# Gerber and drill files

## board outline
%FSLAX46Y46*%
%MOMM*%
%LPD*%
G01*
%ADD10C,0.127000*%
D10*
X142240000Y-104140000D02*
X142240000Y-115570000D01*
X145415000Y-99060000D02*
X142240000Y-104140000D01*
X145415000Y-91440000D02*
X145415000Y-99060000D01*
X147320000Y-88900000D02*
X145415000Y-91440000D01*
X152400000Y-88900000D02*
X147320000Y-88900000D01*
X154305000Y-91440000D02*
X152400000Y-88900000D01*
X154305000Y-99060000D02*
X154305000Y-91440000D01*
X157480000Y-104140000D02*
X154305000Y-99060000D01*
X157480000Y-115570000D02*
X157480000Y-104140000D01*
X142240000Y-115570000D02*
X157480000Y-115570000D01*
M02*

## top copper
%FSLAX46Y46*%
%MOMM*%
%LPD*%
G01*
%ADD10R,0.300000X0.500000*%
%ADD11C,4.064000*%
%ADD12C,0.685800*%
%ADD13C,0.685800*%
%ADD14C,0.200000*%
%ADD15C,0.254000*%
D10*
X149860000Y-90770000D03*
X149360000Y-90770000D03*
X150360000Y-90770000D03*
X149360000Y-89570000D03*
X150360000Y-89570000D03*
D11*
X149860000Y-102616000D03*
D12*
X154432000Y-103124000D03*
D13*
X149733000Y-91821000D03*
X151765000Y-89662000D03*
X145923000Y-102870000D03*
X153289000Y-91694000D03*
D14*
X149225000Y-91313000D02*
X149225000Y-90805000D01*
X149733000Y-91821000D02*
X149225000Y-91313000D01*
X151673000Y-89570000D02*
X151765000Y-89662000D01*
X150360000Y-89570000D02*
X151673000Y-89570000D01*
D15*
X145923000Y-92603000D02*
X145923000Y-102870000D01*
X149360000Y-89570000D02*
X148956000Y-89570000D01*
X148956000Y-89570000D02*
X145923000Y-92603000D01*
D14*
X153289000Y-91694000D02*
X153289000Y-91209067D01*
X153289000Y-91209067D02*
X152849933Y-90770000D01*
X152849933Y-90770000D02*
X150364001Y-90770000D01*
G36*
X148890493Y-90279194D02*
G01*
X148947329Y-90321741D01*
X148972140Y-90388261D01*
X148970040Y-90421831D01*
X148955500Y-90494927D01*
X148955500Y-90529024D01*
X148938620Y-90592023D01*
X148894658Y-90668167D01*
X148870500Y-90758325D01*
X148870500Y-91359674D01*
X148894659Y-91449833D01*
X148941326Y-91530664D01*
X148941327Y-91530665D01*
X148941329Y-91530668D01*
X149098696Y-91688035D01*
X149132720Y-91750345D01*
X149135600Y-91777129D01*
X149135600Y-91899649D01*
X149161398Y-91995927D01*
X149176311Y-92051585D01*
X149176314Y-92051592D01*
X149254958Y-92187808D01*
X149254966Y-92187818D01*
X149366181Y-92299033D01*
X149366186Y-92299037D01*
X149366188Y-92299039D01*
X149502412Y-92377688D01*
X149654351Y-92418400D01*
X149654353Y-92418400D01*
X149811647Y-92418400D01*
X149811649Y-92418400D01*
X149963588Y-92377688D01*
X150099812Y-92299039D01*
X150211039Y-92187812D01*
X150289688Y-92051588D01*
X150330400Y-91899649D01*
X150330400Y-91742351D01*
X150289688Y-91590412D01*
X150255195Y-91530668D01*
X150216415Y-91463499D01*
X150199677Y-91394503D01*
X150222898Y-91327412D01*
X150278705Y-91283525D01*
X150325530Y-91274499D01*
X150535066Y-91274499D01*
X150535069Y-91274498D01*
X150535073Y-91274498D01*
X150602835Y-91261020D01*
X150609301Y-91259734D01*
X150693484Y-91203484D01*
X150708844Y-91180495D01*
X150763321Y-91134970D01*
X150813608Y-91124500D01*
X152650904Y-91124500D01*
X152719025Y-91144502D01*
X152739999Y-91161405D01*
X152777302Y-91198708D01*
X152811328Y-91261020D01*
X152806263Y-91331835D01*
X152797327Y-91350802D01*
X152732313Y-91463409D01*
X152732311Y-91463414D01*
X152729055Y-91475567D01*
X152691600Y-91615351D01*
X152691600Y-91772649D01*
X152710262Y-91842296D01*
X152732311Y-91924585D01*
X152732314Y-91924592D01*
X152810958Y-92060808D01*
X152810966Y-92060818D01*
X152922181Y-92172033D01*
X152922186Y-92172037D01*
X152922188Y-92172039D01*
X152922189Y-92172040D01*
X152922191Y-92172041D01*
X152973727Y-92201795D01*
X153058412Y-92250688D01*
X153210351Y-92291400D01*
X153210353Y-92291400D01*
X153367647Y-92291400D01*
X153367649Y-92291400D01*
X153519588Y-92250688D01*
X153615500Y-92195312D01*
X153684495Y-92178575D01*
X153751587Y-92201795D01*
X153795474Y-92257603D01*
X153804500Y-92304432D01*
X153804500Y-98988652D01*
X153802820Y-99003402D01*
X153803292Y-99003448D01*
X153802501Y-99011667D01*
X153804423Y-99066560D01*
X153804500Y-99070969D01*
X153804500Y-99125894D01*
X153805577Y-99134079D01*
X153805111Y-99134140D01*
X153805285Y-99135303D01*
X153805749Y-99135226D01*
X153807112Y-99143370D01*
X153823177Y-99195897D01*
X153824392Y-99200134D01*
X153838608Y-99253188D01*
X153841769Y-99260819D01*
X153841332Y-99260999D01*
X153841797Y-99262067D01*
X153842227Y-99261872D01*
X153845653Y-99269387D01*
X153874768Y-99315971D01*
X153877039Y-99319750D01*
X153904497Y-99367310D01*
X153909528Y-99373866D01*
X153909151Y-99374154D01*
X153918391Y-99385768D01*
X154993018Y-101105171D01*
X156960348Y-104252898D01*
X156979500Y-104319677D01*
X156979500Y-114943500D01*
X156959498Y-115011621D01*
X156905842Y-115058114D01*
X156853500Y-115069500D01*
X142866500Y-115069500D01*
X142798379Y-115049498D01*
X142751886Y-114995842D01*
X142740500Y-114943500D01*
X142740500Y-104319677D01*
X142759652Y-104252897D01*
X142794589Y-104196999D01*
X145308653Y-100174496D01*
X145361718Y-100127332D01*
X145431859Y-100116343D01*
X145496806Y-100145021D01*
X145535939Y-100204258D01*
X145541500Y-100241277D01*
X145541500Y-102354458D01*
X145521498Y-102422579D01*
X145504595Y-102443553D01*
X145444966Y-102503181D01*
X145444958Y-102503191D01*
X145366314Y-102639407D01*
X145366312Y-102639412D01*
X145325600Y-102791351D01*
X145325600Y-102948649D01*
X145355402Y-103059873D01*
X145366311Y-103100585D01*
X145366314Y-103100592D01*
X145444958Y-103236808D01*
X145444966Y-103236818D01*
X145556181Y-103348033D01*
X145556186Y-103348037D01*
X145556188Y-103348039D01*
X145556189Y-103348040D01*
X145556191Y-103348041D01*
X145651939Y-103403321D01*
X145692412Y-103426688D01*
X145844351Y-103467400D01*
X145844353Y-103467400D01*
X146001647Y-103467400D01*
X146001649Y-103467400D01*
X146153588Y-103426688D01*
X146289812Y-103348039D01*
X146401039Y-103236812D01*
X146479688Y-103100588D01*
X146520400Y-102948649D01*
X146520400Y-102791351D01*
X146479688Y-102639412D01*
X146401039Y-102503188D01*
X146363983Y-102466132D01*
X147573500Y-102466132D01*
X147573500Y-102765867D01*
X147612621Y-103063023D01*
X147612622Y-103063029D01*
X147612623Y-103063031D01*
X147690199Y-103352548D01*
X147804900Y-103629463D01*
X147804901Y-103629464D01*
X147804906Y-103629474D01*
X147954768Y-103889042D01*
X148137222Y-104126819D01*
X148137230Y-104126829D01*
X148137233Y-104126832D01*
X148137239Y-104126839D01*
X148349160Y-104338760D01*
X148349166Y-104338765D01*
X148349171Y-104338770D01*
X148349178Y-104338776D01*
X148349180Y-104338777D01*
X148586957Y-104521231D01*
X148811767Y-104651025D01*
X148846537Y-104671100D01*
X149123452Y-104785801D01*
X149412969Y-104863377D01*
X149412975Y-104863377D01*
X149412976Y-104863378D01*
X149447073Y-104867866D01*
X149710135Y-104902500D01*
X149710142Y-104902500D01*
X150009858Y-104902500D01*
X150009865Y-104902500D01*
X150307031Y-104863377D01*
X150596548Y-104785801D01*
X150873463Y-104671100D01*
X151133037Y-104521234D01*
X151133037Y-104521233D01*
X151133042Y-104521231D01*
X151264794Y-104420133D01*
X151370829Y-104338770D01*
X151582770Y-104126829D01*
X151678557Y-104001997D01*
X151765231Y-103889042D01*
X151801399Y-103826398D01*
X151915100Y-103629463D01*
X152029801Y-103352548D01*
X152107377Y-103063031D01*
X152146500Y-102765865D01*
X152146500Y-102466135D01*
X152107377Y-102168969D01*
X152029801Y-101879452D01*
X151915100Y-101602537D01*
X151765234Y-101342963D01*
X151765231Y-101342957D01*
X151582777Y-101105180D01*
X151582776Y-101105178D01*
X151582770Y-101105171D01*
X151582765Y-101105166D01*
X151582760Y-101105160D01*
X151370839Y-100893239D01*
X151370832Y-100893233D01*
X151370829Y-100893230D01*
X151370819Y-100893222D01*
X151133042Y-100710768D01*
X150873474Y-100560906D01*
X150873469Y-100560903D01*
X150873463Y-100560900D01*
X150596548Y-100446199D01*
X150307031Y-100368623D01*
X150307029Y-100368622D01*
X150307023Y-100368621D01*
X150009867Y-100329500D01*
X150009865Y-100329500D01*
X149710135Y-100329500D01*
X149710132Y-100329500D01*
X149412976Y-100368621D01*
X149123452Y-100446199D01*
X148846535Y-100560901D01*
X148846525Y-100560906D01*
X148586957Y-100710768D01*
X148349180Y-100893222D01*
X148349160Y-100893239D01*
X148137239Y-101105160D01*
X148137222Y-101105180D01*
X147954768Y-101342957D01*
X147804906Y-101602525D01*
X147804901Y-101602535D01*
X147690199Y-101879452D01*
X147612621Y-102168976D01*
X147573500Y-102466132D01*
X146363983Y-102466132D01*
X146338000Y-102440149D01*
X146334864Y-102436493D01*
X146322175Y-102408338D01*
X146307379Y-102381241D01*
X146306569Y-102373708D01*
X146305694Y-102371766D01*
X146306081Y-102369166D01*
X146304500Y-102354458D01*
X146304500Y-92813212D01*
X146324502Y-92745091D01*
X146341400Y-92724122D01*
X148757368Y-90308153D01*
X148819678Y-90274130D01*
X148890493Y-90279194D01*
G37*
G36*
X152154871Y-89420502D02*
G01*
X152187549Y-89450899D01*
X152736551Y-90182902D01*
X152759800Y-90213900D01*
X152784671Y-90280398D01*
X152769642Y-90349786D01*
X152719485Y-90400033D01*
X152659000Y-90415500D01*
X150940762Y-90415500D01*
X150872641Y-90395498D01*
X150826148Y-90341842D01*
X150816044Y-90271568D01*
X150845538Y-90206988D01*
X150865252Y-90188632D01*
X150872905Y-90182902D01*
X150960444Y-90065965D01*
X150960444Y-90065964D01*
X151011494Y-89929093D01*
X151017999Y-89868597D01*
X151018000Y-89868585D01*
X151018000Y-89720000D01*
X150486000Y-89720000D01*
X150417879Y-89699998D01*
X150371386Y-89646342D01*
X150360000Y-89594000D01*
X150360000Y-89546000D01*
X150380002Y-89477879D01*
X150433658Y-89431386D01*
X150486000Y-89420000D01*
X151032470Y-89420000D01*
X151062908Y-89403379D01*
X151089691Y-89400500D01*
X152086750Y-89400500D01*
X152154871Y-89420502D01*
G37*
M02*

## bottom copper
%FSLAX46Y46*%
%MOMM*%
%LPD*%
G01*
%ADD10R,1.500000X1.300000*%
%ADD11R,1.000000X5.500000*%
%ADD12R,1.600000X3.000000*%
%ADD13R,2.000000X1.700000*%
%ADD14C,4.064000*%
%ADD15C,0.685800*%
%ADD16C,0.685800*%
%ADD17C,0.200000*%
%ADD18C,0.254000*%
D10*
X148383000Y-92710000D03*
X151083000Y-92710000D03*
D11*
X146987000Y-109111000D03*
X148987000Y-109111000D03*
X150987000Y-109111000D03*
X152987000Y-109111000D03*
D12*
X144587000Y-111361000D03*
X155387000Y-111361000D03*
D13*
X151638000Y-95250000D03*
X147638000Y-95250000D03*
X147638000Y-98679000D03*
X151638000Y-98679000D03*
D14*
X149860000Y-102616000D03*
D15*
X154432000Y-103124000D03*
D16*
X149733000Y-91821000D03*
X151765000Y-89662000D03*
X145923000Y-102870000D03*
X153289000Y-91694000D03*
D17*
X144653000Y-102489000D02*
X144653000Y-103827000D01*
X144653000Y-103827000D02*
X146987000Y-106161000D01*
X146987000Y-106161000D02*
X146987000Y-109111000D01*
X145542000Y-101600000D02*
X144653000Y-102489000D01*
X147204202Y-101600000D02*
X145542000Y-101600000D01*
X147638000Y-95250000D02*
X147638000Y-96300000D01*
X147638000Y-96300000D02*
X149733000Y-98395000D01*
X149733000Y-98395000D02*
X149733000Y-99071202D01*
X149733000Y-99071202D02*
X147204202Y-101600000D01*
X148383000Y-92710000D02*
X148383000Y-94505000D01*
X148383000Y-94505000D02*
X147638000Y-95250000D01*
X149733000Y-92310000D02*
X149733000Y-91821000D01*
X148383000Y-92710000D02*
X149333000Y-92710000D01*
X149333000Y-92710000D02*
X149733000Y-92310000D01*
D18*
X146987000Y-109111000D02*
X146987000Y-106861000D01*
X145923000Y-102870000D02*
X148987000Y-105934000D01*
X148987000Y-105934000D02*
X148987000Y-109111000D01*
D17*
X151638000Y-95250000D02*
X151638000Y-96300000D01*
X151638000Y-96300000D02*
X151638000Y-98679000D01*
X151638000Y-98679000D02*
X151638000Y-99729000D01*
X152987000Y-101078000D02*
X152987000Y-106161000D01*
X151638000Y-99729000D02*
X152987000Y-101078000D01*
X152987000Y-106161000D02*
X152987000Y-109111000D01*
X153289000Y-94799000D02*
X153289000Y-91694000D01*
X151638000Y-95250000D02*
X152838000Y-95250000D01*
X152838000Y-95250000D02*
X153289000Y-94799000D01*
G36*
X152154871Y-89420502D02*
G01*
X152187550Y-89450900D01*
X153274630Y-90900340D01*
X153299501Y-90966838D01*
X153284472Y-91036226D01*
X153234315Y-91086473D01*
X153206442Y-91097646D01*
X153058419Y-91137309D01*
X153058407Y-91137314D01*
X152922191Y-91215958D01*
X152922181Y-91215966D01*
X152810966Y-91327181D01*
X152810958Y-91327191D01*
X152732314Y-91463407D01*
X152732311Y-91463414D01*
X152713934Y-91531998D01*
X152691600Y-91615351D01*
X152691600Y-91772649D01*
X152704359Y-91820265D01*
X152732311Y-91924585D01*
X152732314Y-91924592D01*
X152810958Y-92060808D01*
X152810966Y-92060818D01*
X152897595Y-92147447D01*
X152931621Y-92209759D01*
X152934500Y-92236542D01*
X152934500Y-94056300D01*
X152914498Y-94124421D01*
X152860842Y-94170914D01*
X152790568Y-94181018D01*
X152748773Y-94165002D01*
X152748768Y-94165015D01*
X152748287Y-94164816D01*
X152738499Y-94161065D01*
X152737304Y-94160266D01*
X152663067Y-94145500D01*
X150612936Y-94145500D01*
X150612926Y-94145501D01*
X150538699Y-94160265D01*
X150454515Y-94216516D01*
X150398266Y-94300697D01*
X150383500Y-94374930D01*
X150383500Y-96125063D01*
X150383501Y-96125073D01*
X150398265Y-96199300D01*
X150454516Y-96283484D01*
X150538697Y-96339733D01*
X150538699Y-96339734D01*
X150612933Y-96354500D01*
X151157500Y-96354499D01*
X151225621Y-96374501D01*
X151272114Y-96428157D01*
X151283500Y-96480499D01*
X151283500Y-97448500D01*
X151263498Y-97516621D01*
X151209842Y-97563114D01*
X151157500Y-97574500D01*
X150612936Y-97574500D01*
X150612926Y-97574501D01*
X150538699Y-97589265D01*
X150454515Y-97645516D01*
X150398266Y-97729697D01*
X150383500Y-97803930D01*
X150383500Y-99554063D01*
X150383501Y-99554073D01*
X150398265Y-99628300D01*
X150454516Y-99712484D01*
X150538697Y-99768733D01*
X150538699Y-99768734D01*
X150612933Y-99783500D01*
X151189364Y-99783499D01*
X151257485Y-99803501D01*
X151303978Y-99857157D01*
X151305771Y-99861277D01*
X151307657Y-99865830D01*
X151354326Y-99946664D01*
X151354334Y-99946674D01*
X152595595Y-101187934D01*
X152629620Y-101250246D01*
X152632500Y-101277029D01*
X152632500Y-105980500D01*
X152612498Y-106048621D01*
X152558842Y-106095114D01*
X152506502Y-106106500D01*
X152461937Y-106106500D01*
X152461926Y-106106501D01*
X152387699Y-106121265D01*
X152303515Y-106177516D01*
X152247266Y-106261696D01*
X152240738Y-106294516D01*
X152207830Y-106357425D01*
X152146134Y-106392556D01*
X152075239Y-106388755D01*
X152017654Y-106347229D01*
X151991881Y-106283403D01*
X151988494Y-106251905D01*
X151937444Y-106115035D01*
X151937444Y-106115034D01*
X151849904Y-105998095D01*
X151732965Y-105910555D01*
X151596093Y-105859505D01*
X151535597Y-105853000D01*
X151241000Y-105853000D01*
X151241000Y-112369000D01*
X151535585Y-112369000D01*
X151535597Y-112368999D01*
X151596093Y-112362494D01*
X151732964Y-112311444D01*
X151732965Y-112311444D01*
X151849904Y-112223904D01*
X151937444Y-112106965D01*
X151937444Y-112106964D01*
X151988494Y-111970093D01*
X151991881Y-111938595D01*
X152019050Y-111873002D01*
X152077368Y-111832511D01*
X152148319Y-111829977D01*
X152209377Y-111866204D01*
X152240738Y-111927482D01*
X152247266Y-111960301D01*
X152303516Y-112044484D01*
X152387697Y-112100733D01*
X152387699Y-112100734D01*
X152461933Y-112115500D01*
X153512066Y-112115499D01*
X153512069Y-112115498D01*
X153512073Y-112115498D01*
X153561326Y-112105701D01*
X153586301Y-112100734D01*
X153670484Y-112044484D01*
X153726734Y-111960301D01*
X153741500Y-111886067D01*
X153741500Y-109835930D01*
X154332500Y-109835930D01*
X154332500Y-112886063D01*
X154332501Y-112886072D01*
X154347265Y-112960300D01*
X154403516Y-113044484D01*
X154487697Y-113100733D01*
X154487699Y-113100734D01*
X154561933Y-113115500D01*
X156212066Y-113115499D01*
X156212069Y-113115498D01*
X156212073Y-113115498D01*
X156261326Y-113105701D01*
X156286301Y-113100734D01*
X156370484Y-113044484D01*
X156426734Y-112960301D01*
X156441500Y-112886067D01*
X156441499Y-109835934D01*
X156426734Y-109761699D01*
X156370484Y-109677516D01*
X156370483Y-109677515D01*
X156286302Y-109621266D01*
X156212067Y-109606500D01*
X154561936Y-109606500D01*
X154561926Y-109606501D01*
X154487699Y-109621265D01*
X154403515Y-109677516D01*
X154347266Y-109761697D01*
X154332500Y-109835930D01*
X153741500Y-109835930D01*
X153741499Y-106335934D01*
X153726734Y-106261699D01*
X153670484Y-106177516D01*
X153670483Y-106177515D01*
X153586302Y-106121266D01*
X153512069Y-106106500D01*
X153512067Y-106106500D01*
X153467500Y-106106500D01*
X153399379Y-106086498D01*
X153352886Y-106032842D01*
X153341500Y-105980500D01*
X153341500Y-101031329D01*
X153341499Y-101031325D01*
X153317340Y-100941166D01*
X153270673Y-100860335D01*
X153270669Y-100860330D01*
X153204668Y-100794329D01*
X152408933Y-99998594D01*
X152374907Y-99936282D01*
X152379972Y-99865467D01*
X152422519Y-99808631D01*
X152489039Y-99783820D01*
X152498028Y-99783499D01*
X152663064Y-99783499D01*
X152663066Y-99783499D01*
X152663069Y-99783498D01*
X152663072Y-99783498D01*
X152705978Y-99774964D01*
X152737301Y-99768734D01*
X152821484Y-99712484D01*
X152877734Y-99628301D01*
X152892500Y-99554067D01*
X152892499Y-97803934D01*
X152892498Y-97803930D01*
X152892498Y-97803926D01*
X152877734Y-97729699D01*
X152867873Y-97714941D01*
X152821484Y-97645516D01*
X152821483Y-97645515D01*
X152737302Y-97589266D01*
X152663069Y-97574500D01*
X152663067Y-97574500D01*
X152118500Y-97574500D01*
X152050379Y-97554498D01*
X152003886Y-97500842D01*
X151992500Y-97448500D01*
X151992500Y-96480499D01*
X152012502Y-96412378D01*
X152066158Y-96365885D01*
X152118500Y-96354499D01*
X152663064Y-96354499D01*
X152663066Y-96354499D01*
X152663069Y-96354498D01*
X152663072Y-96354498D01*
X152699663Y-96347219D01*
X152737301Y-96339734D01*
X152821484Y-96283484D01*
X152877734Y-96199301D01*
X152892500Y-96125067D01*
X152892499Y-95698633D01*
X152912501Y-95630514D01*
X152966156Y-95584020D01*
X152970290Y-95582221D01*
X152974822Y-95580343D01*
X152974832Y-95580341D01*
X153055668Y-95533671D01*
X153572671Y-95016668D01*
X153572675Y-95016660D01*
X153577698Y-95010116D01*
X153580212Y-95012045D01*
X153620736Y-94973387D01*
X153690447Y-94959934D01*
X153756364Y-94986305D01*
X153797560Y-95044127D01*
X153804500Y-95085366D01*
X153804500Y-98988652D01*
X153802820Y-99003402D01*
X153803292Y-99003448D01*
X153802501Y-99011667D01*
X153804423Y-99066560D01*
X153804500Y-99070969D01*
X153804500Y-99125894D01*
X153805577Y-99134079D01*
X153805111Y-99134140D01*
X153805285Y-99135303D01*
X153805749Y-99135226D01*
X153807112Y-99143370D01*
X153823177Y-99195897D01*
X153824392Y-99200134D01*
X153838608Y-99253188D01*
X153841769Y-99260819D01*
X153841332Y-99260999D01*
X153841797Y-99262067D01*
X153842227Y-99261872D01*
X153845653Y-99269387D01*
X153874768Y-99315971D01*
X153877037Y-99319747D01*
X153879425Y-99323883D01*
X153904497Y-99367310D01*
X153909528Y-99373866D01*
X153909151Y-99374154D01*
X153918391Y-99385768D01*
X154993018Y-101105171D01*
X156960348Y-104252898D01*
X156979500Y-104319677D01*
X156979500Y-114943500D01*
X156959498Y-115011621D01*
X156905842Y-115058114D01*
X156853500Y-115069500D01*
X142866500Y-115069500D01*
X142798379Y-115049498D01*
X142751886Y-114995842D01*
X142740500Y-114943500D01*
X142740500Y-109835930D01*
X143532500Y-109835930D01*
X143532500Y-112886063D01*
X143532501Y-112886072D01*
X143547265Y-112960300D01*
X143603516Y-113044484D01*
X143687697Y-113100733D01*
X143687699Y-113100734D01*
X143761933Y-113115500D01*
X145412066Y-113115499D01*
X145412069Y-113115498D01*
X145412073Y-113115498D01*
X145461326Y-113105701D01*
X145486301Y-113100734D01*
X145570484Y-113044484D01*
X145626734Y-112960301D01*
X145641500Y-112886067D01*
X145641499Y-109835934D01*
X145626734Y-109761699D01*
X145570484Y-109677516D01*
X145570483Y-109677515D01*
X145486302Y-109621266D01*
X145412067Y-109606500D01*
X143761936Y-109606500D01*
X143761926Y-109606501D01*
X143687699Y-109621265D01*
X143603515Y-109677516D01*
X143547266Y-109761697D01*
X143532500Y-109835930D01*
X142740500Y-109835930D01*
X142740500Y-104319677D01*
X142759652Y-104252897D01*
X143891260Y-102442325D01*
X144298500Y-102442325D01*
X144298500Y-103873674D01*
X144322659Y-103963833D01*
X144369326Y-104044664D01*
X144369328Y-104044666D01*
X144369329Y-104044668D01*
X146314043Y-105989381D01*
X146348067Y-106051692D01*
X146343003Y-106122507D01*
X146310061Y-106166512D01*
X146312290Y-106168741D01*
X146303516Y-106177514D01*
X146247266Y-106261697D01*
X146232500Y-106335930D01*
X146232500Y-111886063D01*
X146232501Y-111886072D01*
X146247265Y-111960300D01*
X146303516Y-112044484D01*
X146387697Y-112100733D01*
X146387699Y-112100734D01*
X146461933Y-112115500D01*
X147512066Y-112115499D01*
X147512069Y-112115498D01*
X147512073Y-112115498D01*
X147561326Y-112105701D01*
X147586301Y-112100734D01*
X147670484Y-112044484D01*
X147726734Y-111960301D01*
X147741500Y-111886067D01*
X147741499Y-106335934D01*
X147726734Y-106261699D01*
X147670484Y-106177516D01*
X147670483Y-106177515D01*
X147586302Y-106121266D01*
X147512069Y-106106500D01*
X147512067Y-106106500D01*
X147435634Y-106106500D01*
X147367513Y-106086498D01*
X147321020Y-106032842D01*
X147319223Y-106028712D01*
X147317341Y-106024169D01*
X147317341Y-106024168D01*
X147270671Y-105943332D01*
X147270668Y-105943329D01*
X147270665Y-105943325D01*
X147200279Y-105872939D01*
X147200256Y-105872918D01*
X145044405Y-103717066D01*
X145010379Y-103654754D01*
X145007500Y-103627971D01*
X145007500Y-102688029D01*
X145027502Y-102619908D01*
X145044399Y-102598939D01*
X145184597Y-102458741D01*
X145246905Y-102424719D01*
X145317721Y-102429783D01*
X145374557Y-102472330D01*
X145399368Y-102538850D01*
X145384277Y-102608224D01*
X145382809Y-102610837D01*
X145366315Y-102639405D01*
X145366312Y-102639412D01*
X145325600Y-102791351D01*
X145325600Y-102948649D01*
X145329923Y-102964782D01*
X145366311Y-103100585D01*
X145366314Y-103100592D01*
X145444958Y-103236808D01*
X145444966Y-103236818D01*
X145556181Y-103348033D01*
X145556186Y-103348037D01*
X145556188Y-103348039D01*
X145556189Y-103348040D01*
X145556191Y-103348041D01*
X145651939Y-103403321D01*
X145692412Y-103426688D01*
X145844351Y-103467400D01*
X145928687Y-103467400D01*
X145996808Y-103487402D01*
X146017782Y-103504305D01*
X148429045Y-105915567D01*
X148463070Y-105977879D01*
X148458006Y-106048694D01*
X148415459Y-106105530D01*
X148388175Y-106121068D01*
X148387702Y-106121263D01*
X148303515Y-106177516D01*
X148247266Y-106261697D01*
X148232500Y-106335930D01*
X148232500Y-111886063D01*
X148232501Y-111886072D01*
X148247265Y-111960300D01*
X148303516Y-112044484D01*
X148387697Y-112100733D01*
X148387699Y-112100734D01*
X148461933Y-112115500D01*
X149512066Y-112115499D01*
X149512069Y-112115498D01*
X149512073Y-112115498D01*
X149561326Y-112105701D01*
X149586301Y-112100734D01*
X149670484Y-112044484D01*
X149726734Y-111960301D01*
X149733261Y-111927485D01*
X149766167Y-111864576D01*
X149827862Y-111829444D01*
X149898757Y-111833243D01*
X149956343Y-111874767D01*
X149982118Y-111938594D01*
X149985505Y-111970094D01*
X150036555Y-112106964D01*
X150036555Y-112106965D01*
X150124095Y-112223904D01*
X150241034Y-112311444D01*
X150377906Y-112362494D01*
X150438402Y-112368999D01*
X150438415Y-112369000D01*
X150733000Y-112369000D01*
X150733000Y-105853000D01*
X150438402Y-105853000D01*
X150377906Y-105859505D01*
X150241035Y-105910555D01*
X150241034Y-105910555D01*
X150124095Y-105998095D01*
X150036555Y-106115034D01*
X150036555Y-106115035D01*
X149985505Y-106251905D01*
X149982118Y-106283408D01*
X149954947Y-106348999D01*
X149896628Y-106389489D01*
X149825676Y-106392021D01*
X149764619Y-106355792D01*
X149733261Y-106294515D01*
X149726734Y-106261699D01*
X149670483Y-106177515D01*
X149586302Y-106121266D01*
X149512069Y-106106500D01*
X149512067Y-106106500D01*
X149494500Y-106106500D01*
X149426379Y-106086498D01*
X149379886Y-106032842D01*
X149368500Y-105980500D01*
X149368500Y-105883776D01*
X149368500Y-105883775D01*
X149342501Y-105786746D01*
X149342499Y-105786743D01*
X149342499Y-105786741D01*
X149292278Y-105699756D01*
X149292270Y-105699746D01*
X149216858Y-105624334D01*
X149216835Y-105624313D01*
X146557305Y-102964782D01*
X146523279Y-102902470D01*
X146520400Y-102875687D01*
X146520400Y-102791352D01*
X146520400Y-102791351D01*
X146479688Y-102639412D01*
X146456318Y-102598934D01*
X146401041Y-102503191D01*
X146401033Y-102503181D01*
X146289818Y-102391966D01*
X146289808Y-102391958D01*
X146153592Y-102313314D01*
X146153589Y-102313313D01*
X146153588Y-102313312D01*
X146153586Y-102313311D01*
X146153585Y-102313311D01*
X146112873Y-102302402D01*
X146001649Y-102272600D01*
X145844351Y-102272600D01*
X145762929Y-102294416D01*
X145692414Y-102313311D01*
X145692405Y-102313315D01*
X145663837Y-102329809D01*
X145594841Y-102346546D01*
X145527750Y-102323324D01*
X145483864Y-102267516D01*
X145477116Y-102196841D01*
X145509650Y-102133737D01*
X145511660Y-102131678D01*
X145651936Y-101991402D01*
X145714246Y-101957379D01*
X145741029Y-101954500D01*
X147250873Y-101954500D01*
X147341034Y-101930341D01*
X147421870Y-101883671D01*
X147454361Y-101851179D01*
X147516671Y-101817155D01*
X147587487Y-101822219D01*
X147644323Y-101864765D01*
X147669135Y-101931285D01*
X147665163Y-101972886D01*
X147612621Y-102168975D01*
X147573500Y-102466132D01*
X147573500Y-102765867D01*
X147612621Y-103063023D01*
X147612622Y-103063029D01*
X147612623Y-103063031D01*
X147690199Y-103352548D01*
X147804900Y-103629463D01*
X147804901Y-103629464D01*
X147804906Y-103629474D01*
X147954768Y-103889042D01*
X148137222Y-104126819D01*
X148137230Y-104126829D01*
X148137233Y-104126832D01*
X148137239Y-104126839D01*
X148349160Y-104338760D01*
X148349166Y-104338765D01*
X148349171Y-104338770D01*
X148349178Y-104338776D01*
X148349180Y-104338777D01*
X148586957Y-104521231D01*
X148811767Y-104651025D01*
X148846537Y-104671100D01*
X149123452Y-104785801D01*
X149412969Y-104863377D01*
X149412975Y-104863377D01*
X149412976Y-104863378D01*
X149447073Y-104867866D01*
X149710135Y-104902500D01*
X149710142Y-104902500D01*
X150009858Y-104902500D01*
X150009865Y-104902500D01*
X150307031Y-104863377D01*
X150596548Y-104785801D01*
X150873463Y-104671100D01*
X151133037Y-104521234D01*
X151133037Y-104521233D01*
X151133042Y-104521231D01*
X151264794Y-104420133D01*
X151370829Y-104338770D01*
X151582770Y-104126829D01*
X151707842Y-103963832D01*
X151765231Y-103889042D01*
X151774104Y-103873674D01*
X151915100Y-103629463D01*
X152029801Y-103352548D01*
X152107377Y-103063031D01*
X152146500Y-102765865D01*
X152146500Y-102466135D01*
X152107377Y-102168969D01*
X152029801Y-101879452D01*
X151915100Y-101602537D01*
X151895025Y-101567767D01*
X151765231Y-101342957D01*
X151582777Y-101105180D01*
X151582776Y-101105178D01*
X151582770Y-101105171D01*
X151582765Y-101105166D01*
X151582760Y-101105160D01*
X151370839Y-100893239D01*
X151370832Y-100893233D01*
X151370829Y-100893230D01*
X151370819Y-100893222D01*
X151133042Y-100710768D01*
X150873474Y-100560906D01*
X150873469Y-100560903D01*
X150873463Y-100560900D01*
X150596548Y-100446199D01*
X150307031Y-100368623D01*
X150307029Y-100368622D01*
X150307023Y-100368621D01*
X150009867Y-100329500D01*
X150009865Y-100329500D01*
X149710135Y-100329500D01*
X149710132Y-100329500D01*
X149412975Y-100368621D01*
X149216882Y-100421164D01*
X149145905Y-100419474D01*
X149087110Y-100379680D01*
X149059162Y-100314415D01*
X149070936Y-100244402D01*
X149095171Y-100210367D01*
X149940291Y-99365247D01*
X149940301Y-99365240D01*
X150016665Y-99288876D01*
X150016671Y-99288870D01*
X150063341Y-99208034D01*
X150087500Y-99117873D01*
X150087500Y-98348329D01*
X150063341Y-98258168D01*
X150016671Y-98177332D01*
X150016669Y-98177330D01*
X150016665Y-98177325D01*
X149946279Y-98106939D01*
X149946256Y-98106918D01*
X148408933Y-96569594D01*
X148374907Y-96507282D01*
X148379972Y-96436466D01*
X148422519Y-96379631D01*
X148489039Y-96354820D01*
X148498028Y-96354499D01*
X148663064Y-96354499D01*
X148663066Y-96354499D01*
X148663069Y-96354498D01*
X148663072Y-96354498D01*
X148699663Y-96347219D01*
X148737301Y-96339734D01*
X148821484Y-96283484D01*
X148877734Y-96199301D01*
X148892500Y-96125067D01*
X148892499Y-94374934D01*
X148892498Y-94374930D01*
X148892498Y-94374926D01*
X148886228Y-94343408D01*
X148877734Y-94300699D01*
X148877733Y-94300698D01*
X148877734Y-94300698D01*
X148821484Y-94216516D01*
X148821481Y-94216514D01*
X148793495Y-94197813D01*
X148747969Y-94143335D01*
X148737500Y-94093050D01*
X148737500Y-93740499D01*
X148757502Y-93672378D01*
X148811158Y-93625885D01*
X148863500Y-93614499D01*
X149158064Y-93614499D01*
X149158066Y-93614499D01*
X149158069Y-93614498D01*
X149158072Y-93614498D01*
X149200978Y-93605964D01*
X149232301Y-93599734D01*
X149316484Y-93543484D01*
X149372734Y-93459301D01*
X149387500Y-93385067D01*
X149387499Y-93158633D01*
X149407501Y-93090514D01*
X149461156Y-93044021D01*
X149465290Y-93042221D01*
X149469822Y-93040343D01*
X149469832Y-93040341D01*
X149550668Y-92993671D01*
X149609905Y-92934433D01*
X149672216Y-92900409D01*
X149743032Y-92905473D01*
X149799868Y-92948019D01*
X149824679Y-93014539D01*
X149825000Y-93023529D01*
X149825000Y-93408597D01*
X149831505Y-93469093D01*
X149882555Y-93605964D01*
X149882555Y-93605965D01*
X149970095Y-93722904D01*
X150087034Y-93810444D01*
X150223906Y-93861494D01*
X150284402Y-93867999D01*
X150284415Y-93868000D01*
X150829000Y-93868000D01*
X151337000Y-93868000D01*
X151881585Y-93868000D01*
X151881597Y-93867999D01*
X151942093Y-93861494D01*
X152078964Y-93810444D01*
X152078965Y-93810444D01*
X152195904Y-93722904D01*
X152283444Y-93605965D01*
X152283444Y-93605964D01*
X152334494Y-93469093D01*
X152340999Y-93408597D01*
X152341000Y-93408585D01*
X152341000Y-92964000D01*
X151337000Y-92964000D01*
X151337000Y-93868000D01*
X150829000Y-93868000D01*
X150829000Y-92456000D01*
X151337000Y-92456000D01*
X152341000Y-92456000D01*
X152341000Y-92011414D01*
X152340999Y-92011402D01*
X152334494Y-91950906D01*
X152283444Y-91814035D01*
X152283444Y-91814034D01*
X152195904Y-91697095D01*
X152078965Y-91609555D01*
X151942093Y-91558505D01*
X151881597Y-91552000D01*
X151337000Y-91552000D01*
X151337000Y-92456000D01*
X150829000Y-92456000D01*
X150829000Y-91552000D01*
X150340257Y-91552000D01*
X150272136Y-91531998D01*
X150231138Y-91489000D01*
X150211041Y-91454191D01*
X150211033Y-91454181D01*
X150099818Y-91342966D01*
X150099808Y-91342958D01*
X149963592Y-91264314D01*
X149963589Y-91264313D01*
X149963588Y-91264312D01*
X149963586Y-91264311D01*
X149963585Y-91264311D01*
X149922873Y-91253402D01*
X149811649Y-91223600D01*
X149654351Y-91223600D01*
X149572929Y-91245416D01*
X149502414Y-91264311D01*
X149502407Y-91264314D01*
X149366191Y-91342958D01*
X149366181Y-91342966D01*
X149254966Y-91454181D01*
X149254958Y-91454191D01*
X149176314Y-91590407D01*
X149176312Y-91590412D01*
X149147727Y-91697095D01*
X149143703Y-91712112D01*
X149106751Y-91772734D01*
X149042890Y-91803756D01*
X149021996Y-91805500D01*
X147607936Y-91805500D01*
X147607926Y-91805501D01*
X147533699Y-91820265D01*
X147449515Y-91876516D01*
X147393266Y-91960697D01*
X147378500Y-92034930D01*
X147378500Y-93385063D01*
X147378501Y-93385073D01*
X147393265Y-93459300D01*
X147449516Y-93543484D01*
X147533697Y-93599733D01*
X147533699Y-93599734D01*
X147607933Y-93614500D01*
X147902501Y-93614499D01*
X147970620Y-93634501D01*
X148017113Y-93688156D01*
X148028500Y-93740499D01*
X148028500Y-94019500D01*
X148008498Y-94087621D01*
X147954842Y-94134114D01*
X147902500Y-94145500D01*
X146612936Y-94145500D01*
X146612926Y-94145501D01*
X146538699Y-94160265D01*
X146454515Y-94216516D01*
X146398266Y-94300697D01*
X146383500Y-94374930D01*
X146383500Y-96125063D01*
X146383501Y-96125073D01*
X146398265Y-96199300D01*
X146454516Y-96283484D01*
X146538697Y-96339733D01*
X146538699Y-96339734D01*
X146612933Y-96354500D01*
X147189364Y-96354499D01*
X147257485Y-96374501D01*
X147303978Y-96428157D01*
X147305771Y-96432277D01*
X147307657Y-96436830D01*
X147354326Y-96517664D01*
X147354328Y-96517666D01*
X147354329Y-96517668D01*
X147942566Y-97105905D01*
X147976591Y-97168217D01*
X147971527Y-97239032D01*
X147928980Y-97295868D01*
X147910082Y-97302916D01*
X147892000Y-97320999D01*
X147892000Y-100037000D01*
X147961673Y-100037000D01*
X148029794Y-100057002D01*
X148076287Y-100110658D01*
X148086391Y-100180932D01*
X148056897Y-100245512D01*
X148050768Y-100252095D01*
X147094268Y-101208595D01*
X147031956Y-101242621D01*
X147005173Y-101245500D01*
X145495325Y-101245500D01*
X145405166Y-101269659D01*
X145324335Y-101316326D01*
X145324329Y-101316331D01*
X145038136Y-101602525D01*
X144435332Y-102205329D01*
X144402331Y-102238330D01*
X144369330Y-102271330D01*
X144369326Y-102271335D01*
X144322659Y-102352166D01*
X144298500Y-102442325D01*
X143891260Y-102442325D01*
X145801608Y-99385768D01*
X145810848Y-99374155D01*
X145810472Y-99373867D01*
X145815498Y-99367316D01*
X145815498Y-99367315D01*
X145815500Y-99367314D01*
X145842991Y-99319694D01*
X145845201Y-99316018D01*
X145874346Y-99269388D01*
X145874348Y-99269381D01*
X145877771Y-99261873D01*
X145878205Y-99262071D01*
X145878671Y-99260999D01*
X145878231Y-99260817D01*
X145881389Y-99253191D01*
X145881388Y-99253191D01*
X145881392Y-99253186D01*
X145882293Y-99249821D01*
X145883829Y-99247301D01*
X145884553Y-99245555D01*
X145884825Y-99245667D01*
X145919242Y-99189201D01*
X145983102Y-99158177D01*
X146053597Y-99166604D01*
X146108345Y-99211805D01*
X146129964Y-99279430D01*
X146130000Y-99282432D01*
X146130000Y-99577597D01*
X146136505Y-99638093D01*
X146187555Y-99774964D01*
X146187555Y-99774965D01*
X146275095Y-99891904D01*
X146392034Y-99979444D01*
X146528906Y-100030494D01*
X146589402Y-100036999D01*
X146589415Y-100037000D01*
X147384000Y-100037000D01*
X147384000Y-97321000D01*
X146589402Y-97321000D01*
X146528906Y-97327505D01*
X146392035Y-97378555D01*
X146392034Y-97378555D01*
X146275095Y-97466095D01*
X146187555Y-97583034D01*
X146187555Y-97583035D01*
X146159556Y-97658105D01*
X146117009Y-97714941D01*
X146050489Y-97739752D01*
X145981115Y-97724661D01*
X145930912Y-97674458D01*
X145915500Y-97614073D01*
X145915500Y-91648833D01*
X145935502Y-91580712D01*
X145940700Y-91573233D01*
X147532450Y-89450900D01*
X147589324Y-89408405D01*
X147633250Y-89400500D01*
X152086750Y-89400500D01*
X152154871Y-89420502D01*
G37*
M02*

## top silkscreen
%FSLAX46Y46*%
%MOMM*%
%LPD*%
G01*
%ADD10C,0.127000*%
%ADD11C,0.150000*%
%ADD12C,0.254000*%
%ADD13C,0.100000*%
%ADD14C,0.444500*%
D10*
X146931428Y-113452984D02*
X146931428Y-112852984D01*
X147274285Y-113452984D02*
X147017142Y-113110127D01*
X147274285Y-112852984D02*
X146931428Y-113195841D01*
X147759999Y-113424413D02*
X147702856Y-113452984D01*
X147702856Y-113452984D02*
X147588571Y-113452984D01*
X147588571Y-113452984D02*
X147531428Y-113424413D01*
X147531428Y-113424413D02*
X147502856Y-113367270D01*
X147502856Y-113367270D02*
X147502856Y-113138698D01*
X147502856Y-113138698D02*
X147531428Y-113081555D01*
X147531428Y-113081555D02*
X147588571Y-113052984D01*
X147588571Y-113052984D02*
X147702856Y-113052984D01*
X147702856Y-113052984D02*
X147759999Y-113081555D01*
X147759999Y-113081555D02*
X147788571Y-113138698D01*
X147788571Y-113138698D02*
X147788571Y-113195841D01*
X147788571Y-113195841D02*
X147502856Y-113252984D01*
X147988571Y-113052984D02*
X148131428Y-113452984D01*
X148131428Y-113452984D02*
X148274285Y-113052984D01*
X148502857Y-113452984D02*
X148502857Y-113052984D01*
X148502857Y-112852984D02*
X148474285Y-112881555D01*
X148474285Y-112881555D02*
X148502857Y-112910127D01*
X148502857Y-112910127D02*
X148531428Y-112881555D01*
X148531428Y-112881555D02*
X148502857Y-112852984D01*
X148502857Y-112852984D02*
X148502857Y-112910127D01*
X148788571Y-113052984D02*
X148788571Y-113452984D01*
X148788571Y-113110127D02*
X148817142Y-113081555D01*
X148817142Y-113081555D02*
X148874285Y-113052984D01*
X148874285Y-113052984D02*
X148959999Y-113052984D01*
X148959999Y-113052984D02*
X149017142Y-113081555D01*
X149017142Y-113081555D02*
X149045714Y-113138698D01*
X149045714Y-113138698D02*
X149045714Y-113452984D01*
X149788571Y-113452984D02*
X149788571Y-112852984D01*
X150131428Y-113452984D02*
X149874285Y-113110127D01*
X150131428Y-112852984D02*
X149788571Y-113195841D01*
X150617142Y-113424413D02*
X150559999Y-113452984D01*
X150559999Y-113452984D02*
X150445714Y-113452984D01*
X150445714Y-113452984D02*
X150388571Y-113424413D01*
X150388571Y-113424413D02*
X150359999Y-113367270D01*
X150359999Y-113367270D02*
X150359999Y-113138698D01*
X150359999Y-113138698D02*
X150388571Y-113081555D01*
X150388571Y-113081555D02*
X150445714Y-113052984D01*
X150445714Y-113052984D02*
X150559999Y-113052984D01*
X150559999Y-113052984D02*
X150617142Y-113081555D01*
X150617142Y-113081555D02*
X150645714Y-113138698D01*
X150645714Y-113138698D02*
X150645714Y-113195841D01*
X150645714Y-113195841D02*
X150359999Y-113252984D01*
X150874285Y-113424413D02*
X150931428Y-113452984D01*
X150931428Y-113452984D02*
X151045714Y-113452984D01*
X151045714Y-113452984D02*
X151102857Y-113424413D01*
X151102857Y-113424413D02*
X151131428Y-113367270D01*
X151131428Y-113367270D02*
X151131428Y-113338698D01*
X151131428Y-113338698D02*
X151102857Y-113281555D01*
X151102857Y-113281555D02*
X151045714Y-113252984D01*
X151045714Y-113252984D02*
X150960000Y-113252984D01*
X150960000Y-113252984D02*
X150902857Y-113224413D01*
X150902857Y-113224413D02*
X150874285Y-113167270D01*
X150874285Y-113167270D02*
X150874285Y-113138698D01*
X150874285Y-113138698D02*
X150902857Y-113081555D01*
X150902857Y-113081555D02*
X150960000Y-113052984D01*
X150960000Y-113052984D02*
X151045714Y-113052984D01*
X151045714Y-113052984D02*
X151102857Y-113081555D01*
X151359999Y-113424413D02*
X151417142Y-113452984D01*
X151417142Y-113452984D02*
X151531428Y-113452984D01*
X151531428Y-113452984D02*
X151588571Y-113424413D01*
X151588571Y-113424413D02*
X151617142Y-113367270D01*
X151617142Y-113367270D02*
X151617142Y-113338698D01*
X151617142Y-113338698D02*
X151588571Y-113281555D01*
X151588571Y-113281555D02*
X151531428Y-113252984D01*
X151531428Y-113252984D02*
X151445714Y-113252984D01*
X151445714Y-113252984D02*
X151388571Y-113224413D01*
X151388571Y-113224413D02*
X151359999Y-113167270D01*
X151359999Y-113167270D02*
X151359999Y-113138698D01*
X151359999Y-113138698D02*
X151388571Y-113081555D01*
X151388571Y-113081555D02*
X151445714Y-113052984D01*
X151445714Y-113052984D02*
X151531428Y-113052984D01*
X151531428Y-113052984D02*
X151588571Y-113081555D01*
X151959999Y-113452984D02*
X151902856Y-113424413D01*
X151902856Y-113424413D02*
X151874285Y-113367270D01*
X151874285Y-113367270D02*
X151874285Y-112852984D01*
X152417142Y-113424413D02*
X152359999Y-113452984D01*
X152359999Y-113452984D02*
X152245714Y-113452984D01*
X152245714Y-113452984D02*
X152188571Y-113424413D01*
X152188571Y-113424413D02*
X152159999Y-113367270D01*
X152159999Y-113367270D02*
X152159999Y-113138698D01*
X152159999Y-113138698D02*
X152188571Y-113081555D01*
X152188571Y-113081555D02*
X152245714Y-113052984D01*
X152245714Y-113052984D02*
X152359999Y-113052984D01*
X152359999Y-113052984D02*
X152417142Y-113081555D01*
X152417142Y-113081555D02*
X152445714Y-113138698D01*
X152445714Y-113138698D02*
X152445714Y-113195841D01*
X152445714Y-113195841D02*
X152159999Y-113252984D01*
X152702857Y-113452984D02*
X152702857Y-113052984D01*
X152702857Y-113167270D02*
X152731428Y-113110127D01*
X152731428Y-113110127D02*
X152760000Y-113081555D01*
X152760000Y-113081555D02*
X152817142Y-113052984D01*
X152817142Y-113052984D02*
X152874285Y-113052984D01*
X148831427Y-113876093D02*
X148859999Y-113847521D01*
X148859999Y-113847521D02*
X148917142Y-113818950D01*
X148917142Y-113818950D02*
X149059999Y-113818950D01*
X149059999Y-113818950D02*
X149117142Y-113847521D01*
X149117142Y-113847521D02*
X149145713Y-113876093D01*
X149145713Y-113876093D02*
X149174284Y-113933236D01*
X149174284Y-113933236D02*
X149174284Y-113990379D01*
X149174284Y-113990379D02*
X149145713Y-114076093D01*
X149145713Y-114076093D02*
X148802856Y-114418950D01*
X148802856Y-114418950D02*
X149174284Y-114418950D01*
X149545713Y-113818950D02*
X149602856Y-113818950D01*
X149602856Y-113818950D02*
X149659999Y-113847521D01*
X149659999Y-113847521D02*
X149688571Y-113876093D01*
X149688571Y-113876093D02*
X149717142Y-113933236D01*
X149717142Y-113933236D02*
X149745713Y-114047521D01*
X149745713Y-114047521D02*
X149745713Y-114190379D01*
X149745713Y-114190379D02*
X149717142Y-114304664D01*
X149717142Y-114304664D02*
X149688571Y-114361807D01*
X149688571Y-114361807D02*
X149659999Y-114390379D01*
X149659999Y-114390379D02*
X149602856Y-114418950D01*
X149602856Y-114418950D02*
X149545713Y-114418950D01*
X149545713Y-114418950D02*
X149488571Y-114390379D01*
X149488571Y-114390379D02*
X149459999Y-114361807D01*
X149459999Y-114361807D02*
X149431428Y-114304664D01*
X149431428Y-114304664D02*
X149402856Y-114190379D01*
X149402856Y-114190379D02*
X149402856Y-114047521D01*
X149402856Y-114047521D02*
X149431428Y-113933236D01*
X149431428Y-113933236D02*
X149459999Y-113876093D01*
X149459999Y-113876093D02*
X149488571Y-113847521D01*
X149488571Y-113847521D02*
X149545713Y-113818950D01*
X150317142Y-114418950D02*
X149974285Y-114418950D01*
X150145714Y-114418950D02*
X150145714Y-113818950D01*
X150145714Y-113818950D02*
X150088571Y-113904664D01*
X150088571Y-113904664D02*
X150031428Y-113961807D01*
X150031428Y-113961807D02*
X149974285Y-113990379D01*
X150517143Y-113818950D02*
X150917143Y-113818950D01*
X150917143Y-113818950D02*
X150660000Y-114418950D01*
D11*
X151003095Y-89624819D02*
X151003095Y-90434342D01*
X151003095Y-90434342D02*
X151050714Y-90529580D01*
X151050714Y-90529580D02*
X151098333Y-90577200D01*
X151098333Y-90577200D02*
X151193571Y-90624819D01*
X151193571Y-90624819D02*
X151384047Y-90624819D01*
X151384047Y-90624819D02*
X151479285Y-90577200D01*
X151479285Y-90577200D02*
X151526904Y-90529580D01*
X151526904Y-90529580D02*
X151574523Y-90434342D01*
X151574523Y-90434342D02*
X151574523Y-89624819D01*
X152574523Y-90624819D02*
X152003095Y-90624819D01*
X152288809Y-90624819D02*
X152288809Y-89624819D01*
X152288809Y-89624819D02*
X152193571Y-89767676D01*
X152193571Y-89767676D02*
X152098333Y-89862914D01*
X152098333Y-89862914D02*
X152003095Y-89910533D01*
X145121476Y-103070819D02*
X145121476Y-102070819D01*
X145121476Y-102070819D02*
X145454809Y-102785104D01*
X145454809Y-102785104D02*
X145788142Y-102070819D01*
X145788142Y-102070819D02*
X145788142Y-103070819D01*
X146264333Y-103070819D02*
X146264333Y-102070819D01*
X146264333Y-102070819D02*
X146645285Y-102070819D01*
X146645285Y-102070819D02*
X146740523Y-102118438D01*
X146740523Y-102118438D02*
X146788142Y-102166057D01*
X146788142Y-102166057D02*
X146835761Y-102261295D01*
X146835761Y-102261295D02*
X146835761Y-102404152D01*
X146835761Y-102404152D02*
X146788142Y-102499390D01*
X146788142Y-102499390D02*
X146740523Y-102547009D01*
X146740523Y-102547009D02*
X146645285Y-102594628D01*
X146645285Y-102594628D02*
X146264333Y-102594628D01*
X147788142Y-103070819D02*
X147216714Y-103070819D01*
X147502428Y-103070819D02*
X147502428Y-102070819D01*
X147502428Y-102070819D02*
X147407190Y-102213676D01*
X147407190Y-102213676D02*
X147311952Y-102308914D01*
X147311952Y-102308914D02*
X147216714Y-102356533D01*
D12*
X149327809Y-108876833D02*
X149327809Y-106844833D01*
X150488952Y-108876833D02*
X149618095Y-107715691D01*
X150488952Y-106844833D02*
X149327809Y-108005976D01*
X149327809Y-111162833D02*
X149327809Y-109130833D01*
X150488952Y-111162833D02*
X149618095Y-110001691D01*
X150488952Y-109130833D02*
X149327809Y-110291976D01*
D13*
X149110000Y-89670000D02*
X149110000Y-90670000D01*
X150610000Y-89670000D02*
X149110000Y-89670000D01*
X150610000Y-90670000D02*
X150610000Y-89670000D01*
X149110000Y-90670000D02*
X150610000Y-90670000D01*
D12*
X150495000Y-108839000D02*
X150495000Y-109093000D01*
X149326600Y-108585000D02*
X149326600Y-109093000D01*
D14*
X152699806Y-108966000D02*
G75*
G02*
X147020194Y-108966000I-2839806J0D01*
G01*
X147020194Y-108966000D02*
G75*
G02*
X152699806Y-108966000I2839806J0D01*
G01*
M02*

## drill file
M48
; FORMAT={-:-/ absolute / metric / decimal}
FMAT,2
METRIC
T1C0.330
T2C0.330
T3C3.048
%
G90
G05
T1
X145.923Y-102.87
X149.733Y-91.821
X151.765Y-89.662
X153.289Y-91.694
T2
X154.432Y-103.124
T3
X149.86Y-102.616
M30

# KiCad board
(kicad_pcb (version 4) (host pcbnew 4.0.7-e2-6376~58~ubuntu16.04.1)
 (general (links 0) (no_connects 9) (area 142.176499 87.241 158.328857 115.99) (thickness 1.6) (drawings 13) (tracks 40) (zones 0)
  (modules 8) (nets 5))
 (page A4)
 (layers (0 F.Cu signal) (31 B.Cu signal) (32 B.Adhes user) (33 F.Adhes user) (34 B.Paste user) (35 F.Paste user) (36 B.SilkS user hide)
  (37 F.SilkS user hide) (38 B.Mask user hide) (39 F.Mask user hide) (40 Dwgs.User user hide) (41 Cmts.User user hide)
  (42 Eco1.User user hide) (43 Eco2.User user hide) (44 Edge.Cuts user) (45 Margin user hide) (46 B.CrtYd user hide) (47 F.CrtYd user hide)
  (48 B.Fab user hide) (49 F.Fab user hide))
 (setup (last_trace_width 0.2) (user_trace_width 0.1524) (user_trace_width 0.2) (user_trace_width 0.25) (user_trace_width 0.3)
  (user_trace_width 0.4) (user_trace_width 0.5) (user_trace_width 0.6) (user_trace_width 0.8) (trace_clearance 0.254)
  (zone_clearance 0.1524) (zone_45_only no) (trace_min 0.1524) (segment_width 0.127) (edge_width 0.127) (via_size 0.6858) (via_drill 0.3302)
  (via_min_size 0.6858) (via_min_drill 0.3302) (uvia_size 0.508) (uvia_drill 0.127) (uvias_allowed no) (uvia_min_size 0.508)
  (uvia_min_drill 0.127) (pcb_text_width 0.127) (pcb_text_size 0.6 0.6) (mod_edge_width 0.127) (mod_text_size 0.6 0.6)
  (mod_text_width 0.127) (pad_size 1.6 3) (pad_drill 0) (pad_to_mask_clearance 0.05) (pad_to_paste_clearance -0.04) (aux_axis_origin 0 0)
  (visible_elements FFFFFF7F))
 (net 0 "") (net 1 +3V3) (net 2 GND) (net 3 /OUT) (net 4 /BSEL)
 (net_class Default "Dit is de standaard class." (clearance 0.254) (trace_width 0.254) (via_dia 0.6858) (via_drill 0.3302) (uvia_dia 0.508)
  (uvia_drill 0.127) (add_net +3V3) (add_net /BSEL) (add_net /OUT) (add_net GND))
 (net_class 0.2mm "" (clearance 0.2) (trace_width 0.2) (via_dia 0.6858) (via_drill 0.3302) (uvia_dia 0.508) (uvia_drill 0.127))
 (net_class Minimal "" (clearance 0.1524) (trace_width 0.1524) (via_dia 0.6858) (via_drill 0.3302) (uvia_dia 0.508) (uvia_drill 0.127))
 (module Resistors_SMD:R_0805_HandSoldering (layer B.Cu) (at 149.733 92.71)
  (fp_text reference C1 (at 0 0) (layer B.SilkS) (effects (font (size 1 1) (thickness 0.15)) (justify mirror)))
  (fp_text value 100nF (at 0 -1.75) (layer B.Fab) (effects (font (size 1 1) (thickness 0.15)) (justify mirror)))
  (pad 1 smd rect (at -1.35 0) (size 1.5 1.3) (layers B.Cu B.Paste B.Mask) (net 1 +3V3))
  (pad 2 smd rect (at 1.35 0) (size 1.5 1.3) (layers B.Cu B.Paste B.Mask) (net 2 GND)))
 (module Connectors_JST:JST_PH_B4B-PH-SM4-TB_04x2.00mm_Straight (layer B.Cu) (at 149.987 110.236)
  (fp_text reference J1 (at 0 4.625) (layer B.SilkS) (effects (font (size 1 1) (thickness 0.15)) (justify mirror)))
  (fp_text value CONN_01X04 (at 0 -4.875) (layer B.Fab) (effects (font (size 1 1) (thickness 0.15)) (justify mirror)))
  (pad 1 smd rect (at -3 -1.125) (size 1 5.5) (layers B.Cu B.Paste B.Mask) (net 1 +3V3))
  (pad 2 smd rect (at -1 -1.125) (size 1 5.5) (layers B.Cu B.Paste B.Mask) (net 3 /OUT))
  (pad 3 smd rect (at 1 -1.125) (size 1 5.5) (layers B.Cu B.Paste B.Mask) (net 2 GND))
  (pad 4 smd rect (at 3 -1.125) (size 1 5.5) (layers B.Cu B.Paste B.Mask) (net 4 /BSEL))
  (pad "" smd rect (at -5.4 1.125) (size 1.6 3) (layers B.Cu B.Paste B.Mask))
  (pad "" smd rect (at 5.4 1.125) (size 1.6 3) (layers B.Cu B.Paste B.Mask)))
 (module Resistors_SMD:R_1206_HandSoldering (layer B.Cu) (at 149.638 95.25 180)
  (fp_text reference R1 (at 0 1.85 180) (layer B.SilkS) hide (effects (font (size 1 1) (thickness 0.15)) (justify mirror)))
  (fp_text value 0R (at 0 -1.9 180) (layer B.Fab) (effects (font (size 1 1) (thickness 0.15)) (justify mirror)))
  (pad 1 smd rect (at -2 0 180) (size 2 1.7) (layers B.Cu B.Paste B.Mask) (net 4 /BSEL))
  (pad 2 smd rect (at 2 0 180) (size 2 1.7) (layers B.Cu B.Paste B.Mask) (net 1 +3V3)))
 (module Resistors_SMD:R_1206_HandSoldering (layer B.Cu) (at 149.638 98.679)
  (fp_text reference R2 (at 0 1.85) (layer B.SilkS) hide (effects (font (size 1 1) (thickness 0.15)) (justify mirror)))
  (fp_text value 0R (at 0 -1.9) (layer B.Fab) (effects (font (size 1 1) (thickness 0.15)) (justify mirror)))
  (pad 1 smd rect (at -2 0) (size 2 1.7) (layers B.Cu B.Paste B.Mask) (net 2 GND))
  (pad 2 smd rect (at 2 0) (size 2 1.7) (layers B.Cu B.Paste B.Mask) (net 4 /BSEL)))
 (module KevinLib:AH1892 (layer F.Cu) (at 149.86 90.17)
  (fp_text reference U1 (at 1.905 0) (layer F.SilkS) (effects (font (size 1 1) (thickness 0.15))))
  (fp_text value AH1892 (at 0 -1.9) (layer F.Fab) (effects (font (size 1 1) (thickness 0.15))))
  (fp_line (start -0.75 -0.5) (end -0.75 0.5) (layer F.SilkS) (width 0.1))
  (fp_line (start 0.75 -0.5) (end -0.75 -0.5) (layer F.SilkS) (width 0.1))
  (fp_line (start 0.75 0.5) (end 0.75 -0.5) (layer F.SilkS) (width 0.1))
  (fp_line (start -0.75 0.5) (end 0.75 0.5) (layer F.SilkS) (width 0.1))
  (pad 2 smd rect (at 0 0.6) (size 0.3 0.5) (layers F.Cu F.Paste F.Mask))
  (pad 1 smd rect (at -0.5 0.6) (size 0.3 0.5) (layers F.Cu F.Paste F.Mask) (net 1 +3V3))
  (pad 3 smd rect (at 0.5 0.6) (size 0.3 0.5) (layers F.Cu F.Paste F.Mask) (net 4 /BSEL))
  (pad 5 smd rect (at -0.5 -0.6) (size 0.3 0.5) (layers F.Cu F.Paste F.Mask) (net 3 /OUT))
  (pad 4 smd rect (at 0.5 -0.6) (size 0.3 0.5) (layers F.Cu F.Paste F.Mask) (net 2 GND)))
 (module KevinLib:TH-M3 (layer F.Cu) (at 149.86 102.616)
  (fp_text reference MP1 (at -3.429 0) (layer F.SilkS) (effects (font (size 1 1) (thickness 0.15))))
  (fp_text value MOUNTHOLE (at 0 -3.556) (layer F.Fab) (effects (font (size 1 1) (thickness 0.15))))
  (pad "" np_thru_hole circle (at 0 0) (size 4.064 4.064) (drill 3.048) (layers *.Cu *.Mask)))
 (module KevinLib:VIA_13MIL (layer F.Cu) (at 154.432 103.124)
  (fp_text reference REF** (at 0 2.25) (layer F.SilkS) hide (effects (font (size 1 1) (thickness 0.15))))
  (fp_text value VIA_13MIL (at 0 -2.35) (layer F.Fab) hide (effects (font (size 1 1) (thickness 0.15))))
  (pad 1 thru_hole circle (at 0 0) (size 0.6858 0.6858) (drill 0.3302) (layers *.Cu) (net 2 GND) (zone_connect 2)))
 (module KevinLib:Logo (layer F.Cu) (at 149.86 108.966)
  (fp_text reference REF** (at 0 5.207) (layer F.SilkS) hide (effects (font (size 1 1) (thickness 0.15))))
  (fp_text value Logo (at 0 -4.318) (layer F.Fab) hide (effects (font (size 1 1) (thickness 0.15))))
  (fp_line (start 0.635 -0.127) (end 0.635 0.127) (layer F.SilkS) (width 0.254))
  (fp_line (start -0.5334 -0.381) (end -0.5334 0.127) (layer F.SilkS) (width 0.254))
  (fp_circle (center 0 0) (end 2.54 -1.27) (layer F.SilkS) (width 0.4445))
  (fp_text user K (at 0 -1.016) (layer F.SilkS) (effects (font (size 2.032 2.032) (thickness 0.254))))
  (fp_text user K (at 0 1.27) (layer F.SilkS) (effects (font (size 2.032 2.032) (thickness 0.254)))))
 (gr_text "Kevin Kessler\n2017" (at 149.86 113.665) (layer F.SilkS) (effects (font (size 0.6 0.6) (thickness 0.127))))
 (gr_line (start 142.24 104.14) (end 142.24 115.57) (layer Edge.Cuts) (width 0.127))
 (gr_line (start 145.415 99.06) (end 142.24 104.14) (layer Edge.Cuts) (width 0.127))
 (gr_line (start 145.415 91.44) (end 145.415 99.06) (layer Edge.Cuts) (width 0.127))
 (gr_line (start 147.32 88.9) (end 145.415 91.44) (layer Edge.Cuts) (width 0.127))
 (gr_line (start 152.4 88.9) (end 147.32 88.9) (layer Edge.Cuts) (width 0.127))
 (gr_line (start 154.305 91.44) (end 152.4 88.9) (layer Edge.Cuts) (width 0.127))
 (gr_line (start 154.305 99.06) (end 154.305 91.44) (layer Edge.Cuts) (width 0.127))
 (gr_line (start 157.48 104.14) (end 154.305 99.06) (layer Edge.Cuts) (width 0.127))
 (gr_line (start 157.48 115.57) (end 157.48 104.14) (layer Edge.Cuts) (width 0.127))
 (gr_line (start 142.24 115.57) (end 157.48 115.57) (layer Edge.Cuts) (width 0.127))
 (segment (start 144.653 102.489) (end 144.653 103.827) (width 0.2) (layer B.Cu) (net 1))
 (segment (start 144.653 103.827) (end 146.987 106.161) (width 0.2) (layer B.Cu) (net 1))
 (segment (start 146.987 106.161) (end 146.987 109.111) (width 0.2) (layer B.Cu) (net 1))
 (segment (start 145.542 101.6) (end 144.653 102.489) (width 0.2) (layer B.Cu) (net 1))
 (segment (start 147.204202 101.6) (end 145.542 101.6) (width 0.2) (layer B.Cu) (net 1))
 (segment (start 147.638 95.25) (end 147.638 96.3) (width 0.2) (layer B.Cu) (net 1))
 (segment (start 147.638 96.3) (end 149.733 98.395) (width 0.2) (layer B.Cu) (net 1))
 (segment (start 149.733 98.395) (end 149.733 99.071202) (width 0.2) (layer B.Cu) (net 1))
 (segment (start 149.733 99.071202) (end 147.204202 101.6) (width 0.2) (layer B.Cu) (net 1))
 (segment (start 148.383 92.71) (end 148.383 94.505) (width 0.2) (layer B.Cu) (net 1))
 (segment (start 148.383 94.505) (end 147.638 95.25) (width 0.2) (layer B.Cu) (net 1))
 (segment (start 149.225 91.313) (end 149.225 90.805) (width 0.2) (layer F.Cu) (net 1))
 (segment (start 149.733 91.821) (end 149.225 91.313) (width 0.2) (layer F.Cu) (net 1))
 (segment (start 149.733 92.31) (end 149.733 91.821) (width 0.2) (layer B.Cu) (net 1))
 (via (at 149.733 91.821) (size 0.6858) (drill 0.3302) (layers F.Cu B.Cu) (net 1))
 (segment (start 148.383 92.71) (end 149.333 92.71) (width 0.2) (layer B.Cu) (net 1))
 (segment (start 149.333 92.71) (end 149.733 92.31) (width 0.2) (layer B.Cu) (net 1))
 (segment (start 146.987 109.111) (end 146.987 106.861) (width 0.254) (layer B.Cu) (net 1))
 (segment (start 151.673 89.57) (end 151.765 89.662) (width 0.2) (layer F.Cu) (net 2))
 (via (at 151.765 89.662) (size 0.6858) (drill 0.3302) (layers F.Cu B.Cu) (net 2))
 (segment (start 150.36 89.57) (end 151.673 89.57) (width 0.2) (layer F.Cu) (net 2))
 (segment (start 145.923 102.87) (end 148.987 105.934) (width 0.254) (layer B.Cu) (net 3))
 (segment (start 148.987 105.934) (end 148.987 109.111) (width 0.254) (layer B.Cu) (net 3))
 (via (at 145.923 102.87) (size 0.6858) (drill 0.3302) (layers F.Cu B.Cu) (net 3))
 (segment (start 145.923 92.603) (end 145.923 102.87) (width 0.254) (layer F.Cu) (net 3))
 (segment (start 149.36 89.57) (end 148.956 89.57) (width 0.254) (layer F.Cu) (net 3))
 (segment (start 148.956 89.57) (end 145.923 92.603) (width 0.254) (layer F.Cu) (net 3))
 (segment (start 151.638 95.25) (end 151.638 96.3) (width 0.2) (layer B.Cu) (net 4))
 (segment (start 151.638 96.3) (end 151.638 98.679) (width 0.2) (layer B.Cu) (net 4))
 (segment (start 151.638 98.679) (end 151.638 99.729) (width 0.2) (layer B.Cu) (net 4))
 (segment (start 152.987 101.078) (end 152.987 106.161) (width 0.2) (layer B.Cu) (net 4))
 (segment (start 151.638 99.729) (end 152.987 101.078) (width 0.2) (layer B.Cu) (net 4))
 (segment (start 152.987 106.161) (end 152.987 109.111) (width 0.2) (layer B.Cu) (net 4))
 (segment (start 153.289 91.694) (end 153.289 91.209067) (width 0.2) (layer F.Cu) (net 4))
 (segment (start 153.289 91.209067) (end 152.849933 90.77) (width 0.2) (layer F.Cu) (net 4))
 (segment (start 152.849933 90.77) (end 150.364001 90.77) (width 0.2) (layer F.Cu) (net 4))
 (segment (start 153.289 94.799) (end 153.289 91.694) (width 0.2) (layer B.Cu) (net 4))
 (via (at 153.289 91.694) (size 0.6858) (drill 0.3302) (layers F.Cu B.Cu) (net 4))
 (segment (start 151.638 95.25) (end 152.838 95.25) (width 0.2) (layer B.Cu) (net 4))
 (segment (start 152.838 95.25) (end 153.289 94.799) (width 0.2) (layer B.Cu) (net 4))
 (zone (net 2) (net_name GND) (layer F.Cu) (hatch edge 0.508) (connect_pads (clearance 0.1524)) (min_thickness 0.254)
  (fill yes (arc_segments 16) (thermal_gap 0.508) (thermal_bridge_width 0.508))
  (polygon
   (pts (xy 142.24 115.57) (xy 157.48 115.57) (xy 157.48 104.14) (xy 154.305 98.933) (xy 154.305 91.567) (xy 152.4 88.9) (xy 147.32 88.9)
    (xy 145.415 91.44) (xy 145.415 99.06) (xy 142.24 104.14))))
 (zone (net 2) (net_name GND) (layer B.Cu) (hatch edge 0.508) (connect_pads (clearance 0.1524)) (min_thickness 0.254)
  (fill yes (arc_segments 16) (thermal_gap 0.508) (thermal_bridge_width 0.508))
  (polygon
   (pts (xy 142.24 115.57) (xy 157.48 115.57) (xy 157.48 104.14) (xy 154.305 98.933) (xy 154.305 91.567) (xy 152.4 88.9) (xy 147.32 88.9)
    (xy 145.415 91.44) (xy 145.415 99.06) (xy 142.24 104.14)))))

